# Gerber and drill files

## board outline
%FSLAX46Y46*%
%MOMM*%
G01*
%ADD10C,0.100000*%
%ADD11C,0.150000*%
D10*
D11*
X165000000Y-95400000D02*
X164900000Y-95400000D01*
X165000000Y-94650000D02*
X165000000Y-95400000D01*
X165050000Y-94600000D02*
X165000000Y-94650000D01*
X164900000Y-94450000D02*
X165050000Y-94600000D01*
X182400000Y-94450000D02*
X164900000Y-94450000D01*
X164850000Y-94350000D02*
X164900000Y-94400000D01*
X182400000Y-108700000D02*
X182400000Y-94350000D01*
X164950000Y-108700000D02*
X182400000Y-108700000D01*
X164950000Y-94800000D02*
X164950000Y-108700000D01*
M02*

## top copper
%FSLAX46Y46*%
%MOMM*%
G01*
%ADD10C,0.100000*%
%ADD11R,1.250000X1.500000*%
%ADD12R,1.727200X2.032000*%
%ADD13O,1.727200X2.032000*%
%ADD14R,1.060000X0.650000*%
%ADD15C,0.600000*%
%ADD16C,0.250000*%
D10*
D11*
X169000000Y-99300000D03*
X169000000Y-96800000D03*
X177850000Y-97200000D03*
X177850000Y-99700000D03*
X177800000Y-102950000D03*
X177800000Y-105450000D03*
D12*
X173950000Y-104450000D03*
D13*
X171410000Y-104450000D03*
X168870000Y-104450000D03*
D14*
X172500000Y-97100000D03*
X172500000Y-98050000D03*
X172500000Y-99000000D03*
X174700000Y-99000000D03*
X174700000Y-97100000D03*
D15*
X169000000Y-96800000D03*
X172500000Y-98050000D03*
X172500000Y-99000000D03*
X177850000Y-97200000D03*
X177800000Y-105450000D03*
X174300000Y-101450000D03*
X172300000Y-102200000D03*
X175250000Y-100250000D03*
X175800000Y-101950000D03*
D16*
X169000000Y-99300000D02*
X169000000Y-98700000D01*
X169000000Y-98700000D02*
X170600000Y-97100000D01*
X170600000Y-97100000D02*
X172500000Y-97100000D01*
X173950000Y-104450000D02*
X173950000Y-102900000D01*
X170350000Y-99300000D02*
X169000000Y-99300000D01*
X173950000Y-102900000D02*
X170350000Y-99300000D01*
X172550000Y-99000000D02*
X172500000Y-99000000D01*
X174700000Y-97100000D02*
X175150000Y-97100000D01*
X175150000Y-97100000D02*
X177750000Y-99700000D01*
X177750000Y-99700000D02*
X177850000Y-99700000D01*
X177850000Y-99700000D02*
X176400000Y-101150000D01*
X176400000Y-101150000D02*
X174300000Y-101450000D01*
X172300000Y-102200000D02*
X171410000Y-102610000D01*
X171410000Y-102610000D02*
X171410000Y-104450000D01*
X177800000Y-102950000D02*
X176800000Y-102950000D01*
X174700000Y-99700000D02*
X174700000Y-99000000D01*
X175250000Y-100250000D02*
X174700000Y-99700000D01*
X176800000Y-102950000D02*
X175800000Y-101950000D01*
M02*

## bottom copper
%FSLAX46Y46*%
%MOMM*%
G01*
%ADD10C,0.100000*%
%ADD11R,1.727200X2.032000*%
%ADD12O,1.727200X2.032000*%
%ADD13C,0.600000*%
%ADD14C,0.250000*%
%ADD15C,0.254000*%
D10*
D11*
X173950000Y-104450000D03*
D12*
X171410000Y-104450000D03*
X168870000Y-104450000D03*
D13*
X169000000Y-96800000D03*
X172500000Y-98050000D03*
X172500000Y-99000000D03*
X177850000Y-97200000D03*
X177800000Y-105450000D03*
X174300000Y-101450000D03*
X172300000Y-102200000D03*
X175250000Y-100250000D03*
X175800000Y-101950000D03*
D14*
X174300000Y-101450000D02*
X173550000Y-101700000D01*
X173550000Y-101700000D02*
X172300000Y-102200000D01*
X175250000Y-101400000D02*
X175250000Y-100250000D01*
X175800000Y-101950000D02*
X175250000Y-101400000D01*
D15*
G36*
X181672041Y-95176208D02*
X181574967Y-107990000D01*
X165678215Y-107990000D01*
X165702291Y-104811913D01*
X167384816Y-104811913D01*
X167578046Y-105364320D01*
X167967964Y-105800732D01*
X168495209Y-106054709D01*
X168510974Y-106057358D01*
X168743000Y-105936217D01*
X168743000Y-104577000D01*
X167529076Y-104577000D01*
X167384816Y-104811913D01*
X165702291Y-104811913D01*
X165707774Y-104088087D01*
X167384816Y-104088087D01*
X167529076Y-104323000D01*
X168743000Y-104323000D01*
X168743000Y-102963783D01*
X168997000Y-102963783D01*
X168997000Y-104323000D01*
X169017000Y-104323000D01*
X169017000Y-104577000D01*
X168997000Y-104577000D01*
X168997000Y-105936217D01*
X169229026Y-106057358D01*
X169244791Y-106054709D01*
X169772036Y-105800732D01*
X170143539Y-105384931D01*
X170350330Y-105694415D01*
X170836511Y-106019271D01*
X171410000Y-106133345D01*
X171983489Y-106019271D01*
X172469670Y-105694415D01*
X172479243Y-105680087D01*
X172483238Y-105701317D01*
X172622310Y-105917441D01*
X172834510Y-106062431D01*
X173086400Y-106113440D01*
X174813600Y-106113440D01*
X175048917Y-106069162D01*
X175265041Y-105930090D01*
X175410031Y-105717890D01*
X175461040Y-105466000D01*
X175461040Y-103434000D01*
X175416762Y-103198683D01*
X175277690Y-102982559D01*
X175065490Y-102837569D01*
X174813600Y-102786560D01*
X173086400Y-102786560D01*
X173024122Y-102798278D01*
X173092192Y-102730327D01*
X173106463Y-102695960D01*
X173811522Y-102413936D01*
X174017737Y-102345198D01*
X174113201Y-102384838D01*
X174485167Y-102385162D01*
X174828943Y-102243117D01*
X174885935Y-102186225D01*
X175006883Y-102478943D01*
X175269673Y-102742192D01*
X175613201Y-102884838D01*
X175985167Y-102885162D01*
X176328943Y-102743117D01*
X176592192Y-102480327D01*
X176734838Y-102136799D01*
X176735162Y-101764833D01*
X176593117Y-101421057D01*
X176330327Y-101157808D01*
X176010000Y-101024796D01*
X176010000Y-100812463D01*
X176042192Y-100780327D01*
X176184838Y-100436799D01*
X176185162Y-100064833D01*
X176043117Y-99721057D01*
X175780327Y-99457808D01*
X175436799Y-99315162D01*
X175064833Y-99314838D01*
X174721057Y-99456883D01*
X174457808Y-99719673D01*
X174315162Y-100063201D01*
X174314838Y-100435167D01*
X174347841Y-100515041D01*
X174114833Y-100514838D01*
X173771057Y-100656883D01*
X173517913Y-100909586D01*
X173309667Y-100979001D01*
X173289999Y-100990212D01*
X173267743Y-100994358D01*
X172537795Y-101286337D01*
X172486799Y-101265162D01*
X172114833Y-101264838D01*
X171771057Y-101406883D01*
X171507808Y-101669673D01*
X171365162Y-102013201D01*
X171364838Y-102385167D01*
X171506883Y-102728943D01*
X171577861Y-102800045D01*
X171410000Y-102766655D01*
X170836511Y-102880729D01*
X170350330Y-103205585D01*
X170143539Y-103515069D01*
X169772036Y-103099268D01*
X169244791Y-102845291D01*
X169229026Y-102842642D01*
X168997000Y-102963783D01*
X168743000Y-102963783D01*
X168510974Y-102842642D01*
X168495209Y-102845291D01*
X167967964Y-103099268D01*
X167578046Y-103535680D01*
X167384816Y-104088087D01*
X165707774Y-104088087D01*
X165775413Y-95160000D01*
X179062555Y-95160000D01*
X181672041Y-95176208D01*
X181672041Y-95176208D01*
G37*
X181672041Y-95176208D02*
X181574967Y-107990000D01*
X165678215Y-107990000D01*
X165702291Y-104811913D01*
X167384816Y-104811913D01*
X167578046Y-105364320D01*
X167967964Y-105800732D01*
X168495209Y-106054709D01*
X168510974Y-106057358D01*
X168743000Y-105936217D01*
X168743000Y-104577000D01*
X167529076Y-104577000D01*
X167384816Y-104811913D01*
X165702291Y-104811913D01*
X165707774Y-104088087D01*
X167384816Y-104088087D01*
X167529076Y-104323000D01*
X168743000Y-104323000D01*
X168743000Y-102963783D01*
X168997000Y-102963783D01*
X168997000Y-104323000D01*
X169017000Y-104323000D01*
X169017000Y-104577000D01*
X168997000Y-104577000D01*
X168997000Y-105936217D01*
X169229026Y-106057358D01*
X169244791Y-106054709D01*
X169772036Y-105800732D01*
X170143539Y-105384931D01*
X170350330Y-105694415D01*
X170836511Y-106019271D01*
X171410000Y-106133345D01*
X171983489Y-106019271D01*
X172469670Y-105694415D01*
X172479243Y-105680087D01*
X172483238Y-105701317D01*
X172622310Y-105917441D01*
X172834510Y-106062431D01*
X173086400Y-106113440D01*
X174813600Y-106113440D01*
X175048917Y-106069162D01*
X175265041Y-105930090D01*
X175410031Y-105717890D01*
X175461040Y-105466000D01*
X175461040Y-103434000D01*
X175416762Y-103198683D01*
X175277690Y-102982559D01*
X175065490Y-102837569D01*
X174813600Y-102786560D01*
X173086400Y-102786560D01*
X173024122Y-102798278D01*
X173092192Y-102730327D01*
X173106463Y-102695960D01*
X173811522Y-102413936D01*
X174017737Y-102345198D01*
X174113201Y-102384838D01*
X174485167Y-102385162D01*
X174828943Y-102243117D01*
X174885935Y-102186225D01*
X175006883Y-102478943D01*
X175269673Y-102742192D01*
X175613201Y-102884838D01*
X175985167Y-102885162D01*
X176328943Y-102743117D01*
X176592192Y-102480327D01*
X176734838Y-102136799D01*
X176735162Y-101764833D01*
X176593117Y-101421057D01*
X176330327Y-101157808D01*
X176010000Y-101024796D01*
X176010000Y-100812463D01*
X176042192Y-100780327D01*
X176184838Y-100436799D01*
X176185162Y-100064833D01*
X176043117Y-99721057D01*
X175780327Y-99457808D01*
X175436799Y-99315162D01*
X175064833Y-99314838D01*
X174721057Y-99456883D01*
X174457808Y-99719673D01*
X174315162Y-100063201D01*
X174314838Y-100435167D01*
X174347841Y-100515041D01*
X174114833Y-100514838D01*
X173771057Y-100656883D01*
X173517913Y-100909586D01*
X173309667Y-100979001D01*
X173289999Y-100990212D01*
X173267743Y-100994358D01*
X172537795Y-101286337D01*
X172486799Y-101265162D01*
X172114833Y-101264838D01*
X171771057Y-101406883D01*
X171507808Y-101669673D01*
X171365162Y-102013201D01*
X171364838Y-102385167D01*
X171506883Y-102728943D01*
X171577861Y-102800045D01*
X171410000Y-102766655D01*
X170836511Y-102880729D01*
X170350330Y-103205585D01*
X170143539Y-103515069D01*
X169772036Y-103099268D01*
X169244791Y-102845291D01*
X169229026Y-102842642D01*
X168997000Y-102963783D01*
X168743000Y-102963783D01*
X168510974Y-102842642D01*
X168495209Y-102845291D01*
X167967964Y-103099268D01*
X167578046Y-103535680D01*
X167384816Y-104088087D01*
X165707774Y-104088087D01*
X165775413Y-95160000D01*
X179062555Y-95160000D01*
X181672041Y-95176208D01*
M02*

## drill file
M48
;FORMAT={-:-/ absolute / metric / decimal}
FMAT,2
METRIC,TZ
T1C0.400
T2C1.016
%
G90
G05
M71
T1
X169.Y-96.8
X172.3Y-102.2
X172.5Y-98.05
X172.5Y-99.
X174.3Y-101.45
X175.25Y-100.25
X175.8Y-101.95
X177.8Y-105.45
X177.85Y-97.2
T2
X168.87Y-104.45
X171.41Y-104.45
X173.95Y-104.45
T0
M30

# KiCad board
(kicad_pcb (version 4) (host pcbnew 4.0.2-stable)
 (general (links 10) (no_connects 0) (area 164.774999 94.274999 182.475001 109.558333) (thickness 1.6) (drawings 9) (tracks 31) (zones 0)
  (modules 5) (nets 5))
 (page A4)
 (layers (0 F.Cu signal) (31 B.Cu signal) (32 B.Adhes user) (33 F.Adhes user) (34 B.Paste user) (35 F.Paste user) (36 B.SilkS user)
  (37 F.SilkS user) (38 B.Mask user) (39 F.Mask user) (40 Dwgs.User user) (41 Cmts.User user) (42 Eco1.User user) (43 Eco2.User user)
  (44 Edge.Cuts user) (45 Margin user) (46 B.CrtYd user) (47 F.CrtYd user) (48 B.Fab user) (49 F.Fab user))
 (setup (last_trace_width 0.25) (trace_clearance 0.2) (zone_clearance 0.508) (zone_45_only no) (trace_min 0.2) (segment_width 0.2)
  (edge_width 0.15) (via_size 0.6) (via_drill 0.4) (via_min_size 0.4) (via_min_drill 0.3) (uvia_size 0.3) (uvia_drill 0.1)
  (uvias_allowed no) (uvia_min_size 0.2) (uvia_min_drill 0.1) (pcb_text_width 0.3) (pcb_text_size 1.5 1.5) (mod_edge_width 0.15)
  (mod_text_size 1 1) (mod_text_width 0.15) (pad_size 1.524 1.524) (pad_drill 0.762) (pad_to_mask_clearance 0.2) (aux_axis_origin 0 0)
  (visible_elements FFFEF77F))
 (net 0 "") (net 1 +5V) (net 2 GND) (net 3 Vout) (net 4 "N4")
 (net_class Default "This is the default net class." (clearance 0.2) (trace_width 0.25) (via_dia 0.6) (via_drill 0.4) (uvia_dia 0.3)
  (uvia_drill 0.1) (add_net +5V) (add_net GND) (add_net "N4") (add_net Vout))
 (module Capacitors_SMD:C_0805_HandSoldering (layer F.Cu) (at 169 98.05 90)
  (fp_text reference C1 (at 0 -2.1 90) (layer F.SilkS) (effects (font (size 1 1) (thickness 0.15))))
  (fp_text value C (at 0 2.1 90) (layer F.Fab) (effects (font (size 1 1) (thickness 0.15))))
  (pad 1 smd rect (at -1.25 0 90) (size 1.5 1.25) (layers F.Cu F.Paste F.Mask) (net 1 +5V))
  (pad 2 smd rect (at 1.25 0 90) (size 1.5 1.25) (layers F.Cu F.Paste F.Mask) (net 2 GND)))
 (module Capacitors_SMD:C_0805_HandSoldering (layer F.Cu) (at 177.85 98.45 270)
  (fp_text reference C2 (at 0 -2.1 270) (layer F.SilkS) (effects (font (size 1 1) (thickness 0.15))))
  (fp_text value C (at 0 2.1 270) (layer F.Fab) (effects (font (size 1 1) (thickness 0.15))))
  (pad 1 smd rect (at -1.25 0 270) (size 1.5 1.25) (layers F.Cu F.Paste F.Mask) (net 2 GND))
  (pad 2 smd rect (at 1.25 0 270) (size 1.5 1.25) (layers F.Cu F.Paste F.Mask) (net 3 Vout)))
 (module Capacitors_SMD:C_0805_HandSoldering (layer F.Cu) (at 177.8 104.2 270)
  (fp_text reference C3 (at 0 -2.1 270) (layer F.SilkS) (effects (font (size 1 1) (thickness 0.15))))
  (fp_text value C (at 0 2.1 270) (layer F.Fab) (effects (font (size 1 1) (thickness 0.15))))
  (pad 1 smd rect (at -1.25 0 270) (size 1.5 1.25) (layers F.Cu F.Paste F.Mask) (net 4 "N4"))
  (pad 2 smd rect (at 1.25 0 270) (size 1.5 1.25) (layers F.Cu F.Paste F.Mask) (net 2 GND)))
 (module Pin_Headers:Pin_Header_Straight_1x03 (layer F.Cu) (at 173.95 104.45 270)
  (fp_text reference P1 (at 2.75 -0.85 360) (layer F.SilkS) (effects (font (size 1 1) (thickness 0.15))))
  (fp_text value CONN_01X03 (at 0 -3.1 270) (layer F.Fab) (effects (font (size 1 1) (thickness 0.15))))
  (pad 1 thru_hole rect (at 0 0 270) (size 2.032 1.7272) (drill 1.016) (layers *.Cu *.Mask F.SilkS) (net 1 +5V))
  (pad 2 thru_hole oval (at 0 2.54 270) (size 2.032 1.7272) (drill 1.016) (layers *.Cu *.Mask F.SilkS) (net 3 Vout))
  (pad 3 thru_hole oval (at 0 5.08 270) (size 2.032 1.7272) (drill 1.016) (layers *.Cu *.Mask F.SilkS) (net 2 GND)))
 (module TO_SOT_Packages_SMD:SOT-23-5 (layer F.Cu) (at 173.6 98.05)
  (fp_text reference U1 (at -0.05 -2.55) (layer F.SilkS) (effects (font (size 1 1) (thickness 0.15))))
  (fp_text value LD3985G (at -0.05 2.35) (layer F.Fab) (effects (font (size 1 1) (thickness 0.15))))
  (pad 1 smd rect (at -1.1 -0.95) (size 1.06 0.65) (layers F.Cu F.Paste F.Mask) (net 1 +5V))
  (pad 2 smd rect (at -1.1 0) (size 1.06 0.65) (layers F.Cu F.Paste F.Mask) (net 2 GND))
  (pad 3 smd rect (at -1.1 0.95) (size 1.06 0.65) (layers F.Cu F.Paste F.Mask) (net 2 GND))
  (pad 4 smd rect (at 1.1 0.95) (size 1.06 0.65) (layers F.Cu F.Paste F.Mask) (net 4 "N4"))
  (pad 5 smd rect (at 1.1 -0.95) (size 1.06 0.65) (layers F.Cu F.Paste F.Mask) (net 3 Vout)))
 (gr_line (start 165 95.4) (end 164.9 95.4) (angle 90) (layer Edge.Cuts) (width 0.15))
 (gr_line (start 165 94.65) (end 165 95.4) (angle 90) (layer Edge.Cuts) (width 0.15))
 (gr_line (start 165.05 94.6) (end 165 94.65) (angle 90) (layer Edge.Cuts) (width 0.15))
 (gr_line (start 164.9 94.45) (end 165.05 94.6) (angle 90) (layer Edge.Cuts) (width 0.15))
 (gr_line (start 182.4 94.45) (end 164.9 94.45) (angle 90) (layer Edge.Cuts) (width 0.15))
 (gr_line (start 164.85 94.35) (end 164.9 94.4) (angle 90) (layer Edge.Cuts) (width 0.15))
 (gr_line (start 182.4 108.7) (end 182.4 94.35) (angle 90) (layer Edge.Cuts) (width 0.15))
 (gr_line (start 164.95 108.7) (end 182.4 108.7) (angle 90) (layer Edge.Cuts) (width 0.15))
 (gr_line (start 164.95 94.8) (end 164.95 108.7) (angle 90) (layer Edge.Cuts) (width 0.15))
 (segment (start 169 99.3) (end 169 98.7) (width 0.25) (layer F.Cu) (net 1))
 (segment (start 169 98.7) (end 170.6 97.1) (width 0.25) (layer F.Cu) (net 1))
 (segment (start 170.6 97.1) (end 172.5 97.1) (width 0.25) (layer F.Cu) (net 1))
 (segment (start 173.95 104.45) (end 173.95 102.9) (width 0.25) (layer F.Cu) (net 1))
 (segment (start 170.35 99.3) (end 169 99.3) (width 0.25) (layer F.Cu) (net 1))
 (segment (start 173.95 102.9) (end 170.35 99.3) (width 0.25) (layer F.Cu) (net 1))
 (via (at 169 96.8) (size 0.6) (drill 0.4) (layers F.Cu B.Cu) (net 2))
 (via (at 172.5 98.05) (size 0.6) (drill 0.4) (layers F.Cu B.Cu) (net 2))
 (via (at 172.5 99) (size 0.6) (drill 0.4) (layers F.Cu B.Cu) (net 2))
 (segment (start 172.55 99) (end 172.5 99) (width 0.25) (layer F.Cu) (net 2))
 (via (at 177.85 97.2) (size 0.6) (drill 0.4) (layers F.Cu B.Cu) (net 2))
 (via (at 177.8 105.45) (size 0.6) (drill 0.4) (layers F.Cu B.Cu) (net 2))
 (segment (start 174.7 97.1) (end 175.15 97.1) (width 0.25) (layer F.Cu) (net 3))
 (segment (start 175.15 97.1) (end 177.75 99.7) (width 0.25) (layer F.Cu) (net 3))
 (segment (start 177.75 99.7) (end 177.85 99.7) (width 0.25) (layer F.Cu) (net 3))
 (segment (start 177.85 99.7) (end 176.4 101.15) (width 0.25) (layer F.Cu) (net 3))
 (segment (start 176.4 101.15) (end 174.3 101.45) (width 0.25) (layer F.Cu) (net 3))
 (via (at 174.3 101.45) (size 0.6) (drill 0.4) (layers F.Cu B.Cu) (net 3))
 (segment (start 174.3 101.45) (end 173.55 101.7) (width 0.25) (layer B.Cu) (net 3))
 (segment (start 173.55 101.7) (end 172.3 102.2) (width 0.25) (layer B.Cu) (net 3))
 (via (at 172.3 102.2) (size 0.6) (drill 0.4) (layers F.Cu B.Cu) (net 3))
 (segment (start 172.3 102.2) (end 171.41 102.61) (width 0.25) (layer F.Cu) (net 3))
 (segment (start 171.41 102.61) (end 171.41 104.45) (width 0.25) (layer F.Cu) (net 3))
 (segment (start 177.8 102.95) (end 176.8 102.95) (width 0.25) (layer F.Cu) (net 4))
 (segment (start 174.7 99.7) (end 174.7 99) (width 0.25) (layer F.Cu) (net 4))
 (segment (start 175.25 100.25) (end 174.7 99.7) (width 0.25) (layer F.Cu) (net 4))
 (via (at 175.25 100.25) (size 0.6) (drill 0.4) (layers F.Cu B.Cu) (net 4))
 (segment (start 175.25 101.4) (end 175.25 100.25) (width 0.25) (layer B.Cu) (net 4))
 (segment (start 175.8 101.95) (end 175.25 101.4) (width 0.25) (layer B.Cu) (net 4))
 (via (at 175.8 101.95) (size 0.6) (drill 0.4) (layers F.Cu B.Cu) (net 4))
 (segment (start 176.8 102.95) (end 175.8 101.95) (width 0.25) (layer F.Cu) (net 4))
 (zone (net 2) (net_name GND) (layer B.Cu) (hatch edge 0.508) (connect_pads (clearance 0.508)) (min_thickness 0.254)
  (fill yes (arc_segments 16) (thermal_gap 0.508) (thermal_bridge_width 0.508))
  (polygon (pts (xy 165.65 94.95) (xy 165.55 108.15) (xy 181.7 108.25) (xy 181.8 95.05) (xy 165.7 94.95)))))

